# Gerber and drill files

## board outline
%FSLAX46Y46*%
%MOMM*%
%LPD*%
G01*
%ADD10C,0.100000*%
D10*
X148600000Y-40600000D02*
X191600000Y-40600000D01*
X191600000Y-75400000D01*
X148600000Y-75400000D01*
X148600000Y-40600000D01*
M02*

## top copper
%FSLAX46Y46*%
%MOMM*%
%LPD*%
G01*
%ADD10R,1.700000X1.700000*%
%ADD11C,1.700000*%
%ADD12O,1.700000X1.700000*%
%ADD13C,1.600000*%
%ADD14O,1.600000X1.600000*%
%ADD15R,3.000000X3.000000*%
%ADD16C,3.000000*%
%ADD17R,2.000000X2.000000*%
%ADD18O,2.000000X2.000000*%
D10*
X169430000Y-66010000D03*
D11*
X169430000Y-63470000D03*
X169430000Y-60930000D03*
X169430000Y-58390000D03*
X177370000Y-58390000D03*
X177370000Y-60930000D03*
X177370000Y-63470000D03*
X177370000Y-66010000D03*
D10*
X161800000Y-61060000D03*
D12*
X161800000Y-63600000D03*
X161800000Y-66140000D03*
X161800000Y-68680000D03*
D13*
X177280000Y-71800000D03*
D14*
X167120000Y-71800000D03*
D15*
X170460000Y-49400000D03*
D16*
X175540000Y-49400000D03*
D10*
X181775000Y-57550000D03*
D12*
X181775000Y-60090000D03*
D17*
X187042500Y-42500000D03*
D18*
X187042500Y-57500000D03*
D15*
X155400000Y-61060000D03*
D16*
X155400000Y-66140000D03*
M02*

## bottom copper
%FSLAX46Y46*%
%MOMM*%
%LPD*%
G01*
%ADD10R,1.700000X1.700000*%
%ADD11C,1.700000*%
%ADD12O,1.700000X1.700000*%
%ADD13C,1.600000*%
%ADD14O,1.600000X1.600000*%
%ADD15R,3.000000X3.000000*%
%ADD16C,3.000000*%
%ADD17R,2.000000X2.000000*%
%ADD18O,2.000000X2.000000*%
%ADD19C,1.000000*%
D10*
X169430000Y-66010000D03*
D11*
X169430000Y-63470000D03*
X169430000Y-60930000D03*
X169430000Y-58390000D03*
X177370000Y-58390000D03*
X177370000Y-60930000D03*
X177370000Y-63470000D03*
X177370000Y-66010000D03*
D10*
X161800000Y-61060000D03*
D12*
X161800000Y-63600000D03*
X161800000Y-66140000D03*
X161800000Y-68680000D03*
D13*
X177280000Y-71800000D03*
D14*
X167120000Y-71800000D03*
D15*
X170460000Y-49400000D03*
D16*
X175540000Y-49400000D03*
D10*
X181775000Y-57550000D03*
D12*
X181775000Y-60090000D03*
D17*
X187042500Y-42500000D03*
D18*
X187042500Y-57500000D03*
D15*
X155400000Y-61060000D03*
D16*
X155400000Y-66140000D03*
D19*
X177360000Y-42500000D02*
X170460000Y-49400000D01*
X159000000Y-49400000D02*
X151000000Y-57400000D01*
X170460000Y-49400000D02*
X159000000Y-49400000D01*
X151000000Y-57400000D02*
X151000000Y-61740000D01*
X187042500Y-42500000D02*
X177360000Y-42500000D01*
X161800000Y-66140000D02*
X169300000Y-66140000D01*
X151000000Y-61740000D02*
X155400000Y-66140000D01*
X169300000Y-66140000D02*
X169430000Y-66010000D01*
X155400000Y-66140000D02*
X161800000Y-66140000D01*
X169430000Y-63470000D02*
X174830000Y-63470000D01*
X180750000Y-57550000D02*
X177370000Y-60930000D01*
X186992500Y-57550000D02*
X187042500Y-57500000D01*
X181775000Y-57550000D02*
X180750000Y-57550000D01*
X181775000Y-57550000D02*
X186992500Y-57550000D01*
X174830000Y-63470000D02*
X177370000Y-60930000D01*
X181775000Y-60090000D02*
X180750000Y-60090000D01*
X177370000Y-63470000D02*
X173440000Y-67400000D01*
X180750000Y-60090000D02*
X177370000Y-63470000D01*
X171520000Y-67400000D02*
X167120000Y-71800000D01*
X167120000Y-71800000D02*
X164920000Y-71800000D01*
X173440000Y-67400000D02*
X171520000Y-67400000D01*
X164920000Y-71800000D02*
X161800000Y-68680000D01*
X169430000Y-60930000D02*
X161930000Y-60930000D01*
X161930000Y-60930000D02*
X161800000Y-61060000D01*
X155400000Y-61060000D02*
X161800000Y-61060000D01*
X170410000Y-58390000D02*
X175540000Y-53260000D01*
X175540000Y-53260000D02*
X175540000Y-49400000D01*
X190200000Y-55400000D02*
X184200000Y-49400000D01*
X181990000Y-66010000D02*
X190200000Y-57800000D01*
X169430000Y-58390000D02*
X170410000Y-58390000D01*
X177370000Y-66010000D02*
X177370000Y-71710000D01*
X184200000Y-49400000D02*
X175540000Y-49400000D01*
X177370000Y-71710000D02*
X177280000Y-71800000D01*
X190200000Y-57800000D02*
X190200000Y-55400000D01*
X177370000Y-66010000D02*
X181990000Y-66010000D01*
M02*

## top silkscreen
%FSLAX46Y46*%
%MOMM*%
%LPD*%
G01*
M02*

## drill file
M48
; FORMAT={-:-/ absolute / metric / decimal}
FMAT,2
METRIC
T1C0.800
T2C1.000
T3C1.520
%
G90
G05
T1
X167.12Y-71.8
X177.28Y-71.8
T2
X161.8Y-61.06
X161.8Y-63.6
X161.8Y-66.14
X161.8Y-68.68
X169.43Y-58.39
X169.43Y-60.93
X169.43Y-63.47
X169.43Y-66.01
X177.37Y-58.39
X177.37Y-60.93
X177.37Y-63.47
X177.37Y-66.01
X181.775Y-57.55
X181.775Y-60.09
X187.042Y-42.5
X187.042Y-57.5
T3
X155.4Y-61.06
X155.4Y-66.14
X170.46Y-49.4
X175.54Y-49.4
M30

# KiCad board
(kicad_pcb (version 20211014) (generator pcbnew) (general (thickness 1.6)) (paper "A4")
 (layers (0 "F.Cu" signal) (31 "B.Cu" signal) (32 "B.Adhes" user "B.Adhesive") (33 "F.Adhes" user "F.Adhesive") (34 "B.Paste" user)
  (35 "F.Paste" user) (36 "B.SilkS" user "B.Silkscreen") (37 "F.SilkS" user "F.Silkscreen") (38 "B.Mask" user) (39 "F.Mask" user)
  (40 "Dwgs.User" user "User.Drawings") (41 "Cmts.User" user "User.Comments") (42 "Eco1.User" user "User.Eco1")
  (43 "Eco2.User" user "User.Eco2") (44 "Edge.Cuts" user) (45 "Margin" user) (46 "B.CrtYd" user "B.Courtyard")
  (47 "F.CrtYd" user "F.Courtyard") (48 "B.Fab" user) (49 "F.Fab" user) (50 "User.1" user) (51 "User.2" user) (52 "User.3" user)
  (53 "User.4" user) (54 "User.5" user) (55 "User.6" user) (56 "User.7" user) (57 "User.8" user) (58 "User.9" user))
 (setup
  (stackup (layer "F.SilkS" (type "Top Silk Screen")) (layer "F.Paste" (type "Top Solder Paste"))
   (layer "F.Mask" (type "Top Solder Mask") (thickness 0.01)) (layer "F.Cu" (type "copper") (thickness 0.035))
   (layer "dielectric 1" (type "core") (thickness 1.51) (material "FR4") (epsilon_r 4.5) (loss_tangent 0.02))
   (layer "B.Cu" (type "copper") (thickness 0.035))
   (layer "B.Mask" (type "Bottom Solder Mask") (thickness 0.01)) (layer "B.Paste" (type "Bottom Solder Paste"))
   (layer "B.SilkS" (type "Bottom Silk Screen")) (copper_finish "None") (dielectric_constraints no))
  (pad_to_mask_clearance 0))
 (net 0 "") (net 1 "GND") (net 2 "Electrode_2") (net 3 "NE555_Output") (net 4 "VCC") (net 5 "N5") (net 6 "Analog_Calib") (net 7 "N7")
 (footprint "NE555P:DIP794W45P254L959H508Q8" (layer "B.Cu") (at 173.4 62.2)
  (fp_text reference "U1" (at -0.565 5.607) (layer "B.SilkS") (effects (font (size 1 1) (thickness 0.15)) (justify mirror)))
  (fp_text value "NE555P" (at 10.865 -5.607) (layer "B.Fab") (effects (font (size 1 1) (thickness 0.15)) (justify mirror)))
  (pad "1" thru_hole rect locked (at -3.97 3.81) (size 1.7 1.7) (drill 1) (layers *.Cu *.Mask) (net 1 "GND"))
  (pad "2" thru_hole circle locked (at -3.97 1.27) (size 1.7 1.7) (drill 1) (layers *.Cu *.Mask) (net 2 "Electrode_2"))
  (pad "3" thru_hole circle locked (at -3.97 -1.27) (size 1.7 1.7) (drill 1) (layers *.Cu *.Mask) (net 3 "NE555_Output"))
  (pad "4" thru_hole circle locked (at -3.97 -3.81) (size 1.7 1.7) (drill 1) (layers *.Cu *.Mask) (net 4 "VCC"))
  (pad "5" thru_hole circle locked (at 3.97 -3.81) (size 1.7 1.7) (drill 1) (layers *.Cu *.Mask) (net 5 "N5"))
  (pad "6" thru_hole circle locked (at 3.97 -1.27) (size 1.7 1.7) (drill 1) (layers *.Cu *.Mask) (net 2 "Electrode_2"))
  (pad "7" thru_hole circle locked (at 3.97 1.27) (size 1.7 1.7) (drill 1) (layers *.Cu *.Mask) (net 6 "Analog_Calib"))
  (pad "8" thru_hole circle locked (at 3.97 3.81) (size 1.7 1.7) (drill 1) (layers *.Cu *.Mask) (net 4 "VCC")))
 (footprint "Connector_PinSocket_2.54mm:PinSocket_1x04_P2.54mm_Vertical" (layer "B.Cu") (at 161.8 61.06 180)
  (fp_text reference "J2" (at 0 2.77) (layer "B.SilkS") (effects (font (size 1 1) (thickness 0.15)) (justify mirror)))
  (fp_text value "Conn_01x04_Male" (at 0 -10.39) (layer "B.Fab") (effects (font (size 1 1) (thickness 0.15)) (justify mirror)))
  (pad "1" thru_hole rect (at 0 0 180) (size 1.7 1.7) (drill 1) (layers *.Cu *.Mask) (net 3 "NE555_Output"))
  (pad "2" thru_hole oval (at 0 -2.54 180) (size 1.7 1.7) (drill 1) (layers *.Cu *.Mask) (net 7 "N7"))
  (pad "3" thru_hole oval (at 0 -5.08 180) (size 1.7 1.7) (drill 1) (layers *.Cu *.Mask) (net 1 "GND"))
  (pad "4" thru_hole oval (at 0 -7.62 180) (size 1.7 1.7) (drill 1) (layers *.Cu *.Mask) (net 6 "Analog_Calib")))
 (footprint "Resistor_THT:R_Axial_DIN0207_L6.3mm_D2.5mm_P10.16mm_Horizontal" (layer "B.Cu") (at 177.28 71.8 180)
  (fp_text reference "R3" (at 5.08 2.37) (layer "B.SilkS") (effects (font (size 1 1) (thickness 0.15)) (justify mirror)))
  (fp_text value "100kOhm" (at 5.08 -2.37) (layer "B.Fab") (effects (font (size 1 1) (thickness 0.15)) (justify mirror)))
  (pad "1" thru_hole circle (at 0 0 180) (size 1.6 1.6) (drill 0.8) (layers *.Cu *.Mask) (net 4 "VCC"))
  (pad "2" thru_hole oval (at 10.16 0 180) (size 1.6 1.6) (drill 0.8) (layers *.Cu *.Mask) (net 6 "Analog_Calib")))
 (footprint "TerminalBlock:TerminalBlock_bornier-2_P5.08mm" (layer "B.Cu") (at 170.46 49.4)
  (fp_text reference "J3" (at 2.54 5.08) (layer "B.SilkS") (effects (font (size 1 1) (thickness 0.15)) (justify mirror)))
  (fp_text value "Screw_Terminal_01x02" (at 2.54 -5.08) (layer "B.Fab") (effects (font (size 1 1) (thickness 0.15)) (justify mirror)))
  (pad "1" thru_hole rect (at 0 0) (size 3 3) (drill 1.52) (layers *.Cu *.Mask) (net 1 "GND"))
  (pad "2" thru_hole circle (at 5.08 0) (size 3 3) (drill 1.52) (layers *.Cu *.Mask) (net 4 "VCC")))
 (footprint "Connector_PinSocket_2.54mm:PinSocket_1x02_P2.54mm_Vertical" (layer "B.Cu") (at 181.775 57.55 180)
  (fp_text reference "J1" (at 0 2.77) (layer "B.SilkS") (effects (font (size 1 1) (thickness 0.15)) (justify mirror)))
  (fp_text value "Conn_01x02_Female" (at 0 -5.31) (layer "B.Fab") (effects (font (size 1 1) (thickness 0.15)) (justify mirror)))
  (pad "1" thru_hole rect (at 0 0 180) (size 1.7 1.7) (drill 1) (layers *.Cu *.Mask) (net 2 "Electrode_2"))
  (pad "2" thru_hole oval (at 0 -2.54 180) (size 1.7 1.7) (drill 1) (layers *.Cu *.Mask) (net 6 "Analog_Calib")))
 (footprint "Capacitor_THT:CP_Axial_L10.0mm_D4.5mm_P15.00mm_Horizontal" (layer "B.Cu") (at 187.0425 42.5 -90)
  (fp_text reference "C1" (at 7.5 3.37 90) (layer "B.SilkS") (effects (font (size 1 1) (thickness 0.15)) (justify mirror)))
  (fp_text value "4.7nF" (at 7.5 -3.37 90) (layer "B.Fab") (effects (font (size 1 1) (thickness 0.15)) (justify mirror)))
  (pad "1" thru_hole rect (at 0 0 270) (size 2 2) (drill 1) (layers *.Cu *.Mask) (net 1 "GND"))
  (pad "2" thru_hole oval (at 15 0 270) (size 2 2) (drill 1) (layers *.Cu *.Mask) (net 2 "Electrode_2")))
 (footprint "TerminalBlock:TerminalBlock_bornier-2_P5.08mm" (layer "B.Cu") (at 155.4 61.06 -90)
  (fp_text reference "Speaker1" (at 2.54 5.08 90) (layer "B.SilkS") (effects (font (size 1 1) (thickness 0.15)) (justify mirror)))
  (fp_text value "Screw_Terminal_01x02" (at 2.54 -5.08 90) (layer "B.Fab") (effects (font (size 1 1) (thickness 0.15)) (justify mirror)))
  (pad "1" thru_hole rect (at 0 0 270) (size 3 3) (drill 1.52) (layers *.Cu *.Mask) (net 3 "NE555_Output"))
  (pad "2" thru_hole circle (at 5.08 0 270) (size 3 3) (drill 1.52) (layers *.Cu *.Mask) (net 1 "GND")))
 (gr_rect (start 148.6 75.4) (end 191.6 40.6) (layer "Edge.Cuts") (width 0.1) (fill none))
 (segment (start 177.36 42.5) (end 170.46 49.4) (width 1) (layer "B.Cu") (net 1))
 (segment (start 159 49.4) (end 151 57.4) (width 1) (layer "B.Cu") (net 1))
 (segment (start 170.46 49.4) (end 159 49.4) (width 1) (layer "B.Cu") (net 1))
 (segment (start 151 57.4) (end 151 61.74) (width 1) (layer "B.Cu") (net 1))
 (segment (start 187.0425 42.5) (end 177.36 42.5) (width 1) (layer "B.Cu") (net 1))
 (segment (start 161.8 66.14) (end 169.3 66.14) (width 1) (layer "B.Cu") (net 1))
 (segment (start 151 61.74) (end 155.4 66.14) (width 1) (layer "B.Cu") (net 1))
 (segment (start 169.3 66.14) (end 169.43 66.01) (width 1) (layer "B.Cu") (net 1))
 (segment (start 155.4 66.14) (end 161.8 66.14) (width 1) (layer "B.Cu") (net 1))
 (segment (start 169.43 63.47) (end 174.83 63.47) (width 1) (layer "B.Cu") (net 2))
 (segment (start 180.75 57.55) (end 177.37 60.93) (width 1) (layer "B.Cu") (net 2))
 (segment (start 186.9925 57.55) (end 187.0425 57.5) (width 1) (layer "B.Cu") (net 2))
 (segment (start 181.775 57.55) (end 180.75 57.55) (width 1) (layer "B.Cu") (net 2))
 (segment (start 181.775 57.55) (end 186.9925 57.55) (width 1) (layer "B.Cu") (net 2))
 (segment (start 174.83 63.47) (end 177.37 60.93) (width 1) (layer "B.Cu") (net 2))
 (segment (start 181.775 60.09) (end 180.75 60.09) (width 1) (layer "B.Cu") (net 6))
 (segment (start 177.37 63.47) (end 173.44 67.4) (width 1) (layer "B.Cu") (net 6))
 (segment (start 180.75 60.09) (end 177.37 63.47) (width 1) (layer "B.Cu") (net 6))
 (segment (start 171.52 67.4) (end 167.12 71.8) (width 1) (layer "B.Cu") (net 6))
 (segment (start 167.12 71.8) (end 164.92 71.8) (width 1) (layer "B.Cu") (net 6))
 (segment (start 173.44 67.4) (end 171.52 67.4) (width 1) (layer "B.Cu") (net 6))
 (segment (start 164.92 71.8) (end 161.8 68.68) (width 1) (layer "B.Cu") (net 6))
 (segment (start 169.43 60.93) (end 161.93 60.93) (width 1) (layer "B.Cu") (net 3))
 (segment (start 161.93 60.93) (end 161.8 61.06) (width 1) (layer "B.Cu") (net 3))
 (segment (start 155.4 61.06) (end 161.8 61.06) (width 1) (layer "B.Cu") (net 3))
 (segment (start 170.41 58.39) (end 175.54 53.26) (width 1) (layer "B.Cu") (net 4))
 (segment (start 175.54 53.26) (end 175.54 49.4) (width 1) (layer "B.Cu") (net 4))
 (segment (start 190.2 55.4) (end 184.2 49.4) (width 1) (layer "B.Cu") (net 4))
 (segment (start 181.99 66.01) (end 190.2 57.8) (width 1) (layer "B.Cu") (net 4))
 (segment (start 169.43 58.39) (end 170.41 58.39) (width 1) (layer "B.Cu") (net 4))
 (segment (start 177.37 66.01) (end 177.37 71.71) (width 1) (layer "B.Cu") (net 4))
 (segment (start 184.2 49.4) (end 175.54 49.4) (width 1) (layer "B.Cu") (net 4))
 (segment (start 177.37 71.71) (end 177.28 71.8) (width 1) (layer "B.Cu") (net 4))
 (segment (start 190.2 57.8) (end 190.2 55.4) (width 1) (layer "B.Cu") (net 4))
 (segment (start 177.37 66.01) (end 181.99 66.01) (width 1) (layer "B.Cu") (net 4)))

